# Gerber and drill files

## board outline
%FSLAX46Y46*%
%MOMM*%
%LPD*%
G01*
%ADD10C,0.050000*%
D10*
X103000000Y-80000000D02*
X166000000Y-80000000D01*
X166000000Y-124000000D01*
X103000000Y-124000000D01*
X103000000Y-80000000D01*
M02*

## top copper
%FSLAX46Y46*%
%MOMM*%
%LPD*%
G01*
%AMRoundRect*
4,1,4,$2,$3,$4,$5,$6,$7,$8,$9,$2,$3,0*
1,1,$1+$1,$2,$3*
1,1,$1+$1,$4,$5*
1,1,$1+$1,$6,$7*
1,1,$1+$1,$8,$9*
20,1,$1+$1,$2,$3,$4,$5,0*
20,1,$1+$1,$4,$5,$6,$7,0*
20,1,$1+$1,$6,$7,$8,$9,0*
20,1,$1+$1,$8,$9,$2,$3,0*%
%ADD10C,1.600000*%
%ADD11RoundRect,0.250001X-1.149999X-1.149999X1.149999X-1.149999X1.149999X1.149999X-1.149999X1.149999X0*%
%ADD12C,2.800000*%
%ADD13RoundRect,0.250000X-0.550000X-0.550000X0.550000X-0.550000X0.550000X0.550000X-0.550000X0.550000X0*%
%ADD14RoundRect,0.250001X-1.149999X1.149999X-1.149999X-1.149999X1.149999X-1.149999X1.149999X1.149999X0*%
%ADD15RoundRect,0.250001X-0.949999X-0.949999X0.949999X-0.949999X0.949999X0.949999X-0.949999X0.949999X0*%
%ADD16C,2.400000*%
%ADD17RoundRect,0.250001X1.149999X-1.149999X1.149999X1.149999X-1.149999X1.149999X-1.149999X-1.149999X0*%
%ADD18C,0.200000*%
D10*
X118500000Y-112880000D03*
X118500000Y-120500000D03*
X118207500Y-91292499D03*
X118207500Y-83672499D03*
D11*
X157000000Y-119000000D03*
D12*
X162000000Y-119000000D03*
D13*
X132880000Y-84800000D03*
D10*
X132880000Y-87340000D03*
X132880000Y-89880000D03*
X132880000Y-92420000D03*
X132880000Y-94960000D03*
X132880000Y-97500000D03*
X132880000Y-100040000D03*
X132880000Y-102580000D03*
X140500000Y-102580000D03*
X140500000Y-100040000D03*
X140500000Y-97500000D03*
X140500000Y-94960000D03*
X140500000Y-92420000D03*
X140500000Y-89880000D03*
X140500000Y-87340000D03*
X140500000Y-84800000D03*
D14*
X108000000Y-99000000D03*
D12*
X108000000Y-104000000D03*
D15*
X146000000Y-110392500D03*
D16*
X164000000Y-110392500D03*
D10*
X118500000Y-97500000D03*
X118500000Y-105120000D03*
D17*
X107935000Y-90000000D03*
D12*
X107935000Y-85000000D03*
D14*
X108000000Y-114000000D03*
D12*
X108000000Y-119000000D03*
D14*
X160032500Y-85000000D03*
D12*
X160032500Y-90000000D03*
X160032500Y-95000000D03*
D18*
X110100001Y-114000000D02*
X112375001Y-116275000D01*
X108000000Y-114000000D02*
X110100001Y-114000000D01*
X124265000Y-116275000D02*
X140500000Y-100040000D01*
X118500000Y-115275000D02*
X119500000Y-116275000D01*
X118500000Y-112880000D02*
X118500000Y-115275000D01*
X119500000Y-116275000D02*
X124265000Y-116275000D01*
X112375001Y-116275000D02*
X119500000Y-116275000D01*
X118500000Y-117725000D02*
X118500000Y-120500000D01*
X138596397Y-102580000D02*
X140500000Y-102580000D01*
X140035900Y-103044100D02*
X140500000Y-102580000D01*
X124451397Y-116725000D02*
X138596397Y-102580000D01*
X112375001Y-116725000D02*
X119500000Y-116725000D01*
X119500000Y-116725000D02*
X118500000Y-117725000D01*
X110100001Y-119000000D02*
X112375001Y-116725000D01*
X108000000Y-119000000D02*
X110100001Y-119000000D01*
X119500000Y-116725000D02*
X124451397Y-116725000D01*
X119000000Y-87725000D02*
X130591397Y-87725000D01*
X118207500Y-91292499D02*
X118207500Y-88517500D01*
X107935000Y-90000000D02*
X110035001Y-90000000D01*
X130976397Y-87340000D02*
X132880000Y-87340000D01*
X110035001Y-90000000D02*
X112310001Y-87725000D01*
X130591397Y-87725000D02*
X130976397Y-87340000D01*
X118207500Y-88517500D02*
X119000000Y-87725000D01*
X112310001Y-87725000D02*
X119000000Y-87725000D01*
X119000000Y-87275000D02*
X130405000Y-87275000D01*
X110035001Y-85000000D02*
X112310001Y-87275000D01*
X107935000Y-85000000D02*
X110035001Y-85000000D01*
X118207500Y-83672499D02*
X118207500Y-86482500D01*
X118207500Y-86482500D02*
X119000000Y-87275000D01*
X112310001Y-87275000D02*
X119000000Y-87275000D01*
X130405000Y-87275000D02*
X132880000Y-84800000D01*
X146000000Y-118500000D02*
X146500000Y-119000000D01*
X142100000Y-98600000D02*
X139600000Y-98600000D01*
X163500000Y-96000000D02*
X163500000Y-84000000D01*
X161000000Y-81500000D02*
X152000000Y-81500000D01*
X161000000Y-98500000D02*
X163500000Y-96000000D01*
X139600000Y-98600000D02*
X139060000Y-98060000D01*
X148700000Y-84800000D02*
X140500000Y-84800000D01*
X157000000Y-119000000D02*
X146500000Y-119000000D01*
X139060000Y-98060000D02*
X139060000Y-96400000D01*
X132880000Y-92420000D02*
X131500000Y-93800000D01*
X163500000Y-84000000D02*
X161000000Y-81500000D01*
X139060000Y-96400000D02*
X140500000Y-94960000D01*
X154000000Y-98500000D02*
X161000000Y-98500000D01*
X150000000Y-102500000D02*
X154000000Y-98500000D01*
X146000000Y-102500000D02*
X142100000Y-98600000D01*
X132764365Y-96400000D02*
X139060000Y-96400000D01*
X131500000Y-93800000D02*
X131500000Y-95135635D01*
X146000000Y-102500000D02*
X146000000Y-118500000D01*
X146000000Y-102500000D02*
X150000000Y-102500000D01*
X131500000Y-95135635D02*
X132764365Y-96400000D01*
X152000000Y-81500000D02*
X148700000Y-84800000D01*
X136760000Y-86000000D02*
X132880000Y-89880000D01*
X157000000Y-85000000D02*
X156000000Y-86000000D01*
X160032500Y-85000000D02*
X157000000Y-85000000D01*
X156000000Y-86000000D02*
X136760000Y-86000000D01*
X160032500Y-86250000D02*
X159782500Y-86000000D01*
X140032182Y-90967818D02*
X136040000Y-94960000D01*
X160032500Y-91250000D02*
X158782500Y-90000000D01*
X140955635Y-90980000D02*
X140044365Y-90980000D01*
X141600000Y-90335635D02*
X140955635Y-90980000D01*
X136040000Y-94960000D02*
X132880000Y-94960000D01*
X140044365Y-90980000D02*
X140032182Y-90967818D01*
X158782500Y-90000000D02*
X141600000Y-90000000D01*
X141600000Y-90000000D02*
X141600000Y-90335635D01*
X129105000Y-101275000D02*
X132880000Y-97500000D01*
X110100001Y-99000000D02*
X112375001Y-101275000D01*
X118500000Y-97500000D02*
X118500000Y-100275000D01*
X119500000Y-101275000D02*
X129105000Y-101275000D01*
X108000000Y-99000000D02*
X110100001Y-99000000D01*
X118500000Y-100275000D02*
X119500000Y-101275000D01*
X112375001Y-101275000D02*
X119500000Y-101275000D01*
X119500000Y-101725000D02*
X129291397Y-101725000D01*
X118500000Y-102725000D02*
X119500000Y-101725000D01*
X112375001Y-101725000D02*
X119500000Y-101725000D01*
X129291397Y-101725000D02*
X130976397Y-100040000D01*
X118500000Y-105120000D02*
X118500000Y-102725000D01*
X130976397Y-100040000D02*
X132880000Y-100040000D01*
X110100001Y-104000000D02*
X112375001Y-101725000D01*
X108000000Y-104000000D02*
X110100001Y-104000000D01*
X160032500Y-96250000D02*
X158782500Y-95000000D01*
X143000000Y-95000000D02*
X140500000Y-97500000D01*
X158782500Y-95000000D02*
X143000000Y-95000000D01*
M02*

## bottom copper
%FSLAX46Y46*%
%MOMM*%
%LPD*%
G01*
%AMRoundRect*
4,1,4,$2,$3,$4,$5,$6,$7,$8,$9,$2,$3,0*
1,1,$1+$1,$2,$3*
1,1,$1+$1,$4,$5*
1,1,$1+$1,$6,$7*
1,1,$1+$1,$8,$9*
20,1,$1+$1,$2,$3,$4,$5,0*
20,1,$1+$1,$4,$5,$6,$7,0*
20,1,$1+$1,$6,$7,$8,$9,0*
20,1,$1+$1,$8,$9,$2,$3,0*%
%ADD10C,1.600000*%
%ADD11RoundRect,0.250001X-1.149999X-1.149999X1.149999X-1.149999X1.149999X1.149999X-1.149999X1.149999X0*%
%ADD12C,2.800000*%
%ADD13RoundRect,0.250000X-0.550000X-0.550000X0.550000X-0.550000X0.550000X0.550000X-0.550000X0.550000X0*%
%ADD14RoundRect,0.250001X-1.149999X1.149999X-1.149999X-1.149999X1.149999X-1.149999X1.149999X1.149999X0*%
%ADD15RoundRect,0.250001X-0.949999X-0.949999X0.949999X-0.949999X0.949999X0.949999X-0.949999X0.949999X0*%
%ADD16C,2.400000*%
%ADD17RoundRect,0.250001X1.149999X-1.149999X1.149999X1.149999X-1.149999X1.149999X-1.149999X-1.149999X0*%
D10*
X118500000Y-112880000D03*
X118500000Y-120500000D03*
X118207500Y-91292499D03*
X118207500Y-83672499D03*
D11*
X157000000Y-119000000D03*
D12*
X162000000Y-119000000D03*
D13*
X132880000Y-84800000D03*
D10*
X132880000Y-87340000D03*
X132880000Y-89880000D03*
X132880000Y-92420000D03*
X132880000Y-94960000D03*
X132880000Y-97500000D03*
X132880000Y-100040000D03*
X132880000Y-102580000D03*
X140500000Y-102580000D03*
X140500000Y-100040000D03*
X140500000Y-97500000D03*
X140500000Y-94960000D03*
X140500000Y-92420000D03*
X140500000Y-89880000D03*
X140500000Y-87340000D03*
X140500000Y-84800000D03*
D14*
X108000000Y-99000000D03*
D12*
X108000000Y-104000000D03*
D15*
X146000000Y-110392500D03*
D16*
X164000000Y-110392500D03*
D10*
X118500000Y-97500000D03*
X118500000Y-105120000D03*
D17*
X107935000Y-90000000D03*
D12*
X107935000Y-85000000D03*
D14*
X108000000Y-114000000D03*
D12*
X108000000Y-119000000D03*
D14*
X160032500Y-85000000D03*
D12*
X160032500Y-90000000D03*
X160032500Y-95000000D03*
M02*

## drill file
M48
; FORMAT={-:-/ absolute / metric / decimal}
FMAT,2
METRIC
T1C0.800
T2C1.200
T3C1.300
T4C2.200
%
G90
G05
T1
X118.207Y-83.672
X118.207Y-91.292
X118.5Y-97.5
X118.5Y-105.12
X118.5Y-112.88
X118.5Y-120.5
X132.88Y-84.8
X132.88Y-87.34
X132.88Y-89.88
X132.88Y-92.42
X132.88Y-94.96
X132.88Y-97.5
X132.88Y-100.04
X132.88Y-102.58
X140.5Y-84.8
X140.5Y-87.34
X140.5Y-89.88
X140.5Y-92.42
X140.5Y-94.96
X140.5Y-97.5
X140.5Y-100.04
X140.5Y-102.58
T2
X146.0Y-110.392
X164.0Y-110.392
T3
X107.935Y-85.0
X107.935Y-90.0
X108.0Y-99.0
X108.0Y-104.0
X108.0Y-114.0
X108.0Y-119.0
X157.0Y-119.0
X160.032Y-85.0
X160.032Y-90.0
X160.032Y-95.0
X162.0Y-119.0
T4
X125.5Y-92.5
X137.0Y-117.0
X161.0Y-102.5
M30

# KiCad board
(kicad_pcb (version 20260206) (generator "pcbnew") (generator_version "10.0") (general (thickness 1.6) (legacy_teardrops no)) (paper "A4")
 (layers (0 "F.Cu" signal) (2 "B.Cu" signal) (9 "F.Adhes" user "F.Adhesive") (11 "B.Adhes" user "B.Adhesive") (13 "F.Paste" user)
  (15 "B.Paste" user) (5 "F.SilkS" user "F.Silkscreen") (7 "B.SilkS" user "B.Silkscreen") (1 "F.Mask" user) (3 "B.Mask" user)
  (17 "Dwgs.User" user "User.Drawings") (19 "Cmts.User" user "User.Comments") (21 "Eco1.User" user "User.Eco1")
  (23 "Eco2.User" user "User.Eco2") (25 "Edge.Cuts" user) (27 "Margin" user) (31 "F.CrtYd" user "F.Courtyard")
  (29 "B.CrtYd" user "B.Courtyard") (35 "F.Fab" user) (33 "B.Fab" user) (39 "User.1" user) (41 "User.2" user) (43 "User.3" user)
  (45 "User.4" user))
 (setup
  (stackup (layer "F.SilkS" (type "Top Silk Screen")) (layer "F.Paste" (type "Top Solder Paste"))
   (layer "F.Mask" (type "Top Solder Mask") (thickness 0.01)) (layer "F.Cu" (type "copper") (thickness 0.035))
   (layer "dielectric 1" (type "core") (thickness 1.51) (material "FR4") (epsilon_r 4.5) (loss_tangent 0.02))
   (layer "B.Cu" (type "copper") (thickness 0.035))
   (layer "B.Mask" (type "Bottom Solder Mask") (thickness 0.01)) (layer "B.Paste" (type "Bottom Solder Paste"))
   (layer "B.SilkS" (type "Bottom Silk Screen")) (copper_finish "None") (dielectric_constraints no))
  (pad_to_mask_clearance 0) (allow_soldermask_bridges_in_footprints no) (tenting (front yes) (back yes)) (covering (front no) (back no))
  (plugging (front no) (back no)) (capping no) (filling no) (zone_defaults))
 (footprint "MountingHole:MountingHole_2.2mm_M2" (layer "F.Cu") (at 125.5 92.5)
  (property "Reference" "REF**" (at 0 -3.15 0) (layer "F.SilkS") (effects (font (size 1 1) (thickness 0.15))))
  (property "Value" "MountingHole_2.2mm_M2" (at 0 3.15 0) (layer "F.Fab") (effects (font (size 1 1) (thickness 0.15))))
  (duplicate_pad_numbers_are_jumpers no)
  (pad "" np_thru_hole circle (at 0 0) (size 2.2 2.2) (drill 2.2) (layers "*.Cu" "*.Mask")))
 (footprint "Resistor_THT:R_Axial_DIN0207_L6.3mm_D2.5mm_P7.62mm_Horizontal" (layer "F.Cu") (at 118.5 112.88 -90)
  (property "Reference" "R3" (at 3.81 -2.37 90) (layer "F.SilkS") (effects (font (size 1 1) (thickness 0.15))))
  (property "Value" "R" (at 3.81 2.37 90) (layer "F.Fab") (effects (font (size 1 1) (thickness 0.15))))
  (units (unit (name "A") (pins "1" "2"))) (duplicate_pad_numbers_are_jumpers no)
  (pad "1" thru_hole circle (at 0 0 270) (size 1.6 1.6) (drill 0.8) (layers "*.Cu" "*.Mask") (remove_unused_layers no) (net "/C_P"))
  (pad "2" thru_hole circle (at 7.62 0 270) (size 1.6 1.6) (drill 0.8) (layers "*.Cu" "*.Mask") (remove_unused_layers no) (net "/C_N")))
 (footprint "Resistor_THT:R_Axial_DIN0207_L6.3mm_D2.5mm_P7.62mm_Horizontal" (layer "F.Cu") (at 118.2075 91.292499 90)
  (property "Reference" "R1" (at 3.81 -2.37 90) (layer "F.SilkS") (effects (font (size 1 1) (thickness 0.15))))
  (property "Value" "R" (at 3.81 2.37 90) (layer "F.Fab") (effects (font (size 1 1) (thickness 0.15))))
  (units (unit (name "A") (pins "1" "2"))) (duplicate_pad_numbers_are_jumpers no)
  (pad "1" thru_hole circle (at 0 0 90) (size 1.6 1.6) (drill 0.8) (layers "*.Cu" "*.Mask") (remove_unused_layers no) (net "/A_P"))
  (pad "2" thru_hole circle (at 7.62 0 90) (size 1.6 1.6) (drill 0.8) (layers "*.Cu" "*.Mask") (remove_unused_layers no) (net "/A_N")))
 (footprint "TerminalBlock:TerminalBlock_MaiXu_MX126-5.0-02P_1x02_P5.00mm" (layer "F.Cu") (at 157 119)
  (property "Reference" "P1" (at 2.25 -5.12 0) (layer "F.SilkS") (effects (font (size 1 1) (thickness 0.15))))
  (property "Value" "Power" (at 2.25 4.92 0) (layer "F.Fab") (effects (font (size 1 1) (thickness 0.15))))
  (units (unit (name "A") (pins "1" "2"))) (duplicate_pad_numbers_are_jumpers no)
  (pad "1" thru_hole roundrect (at 0 0) (size 2.8 2.8) (drill 1.3) (layers "*.Cu" "*.Mask") (remove_unused_layers no)
   (roundrect_rratio 0.089286) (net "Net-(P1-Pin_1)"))
  (pad "2" thru_hole circle (at 5 0) (size 2.8 2.8) (drill 1.3) (layers "*.Cu" "*.Mask") (remove_unused_layers no) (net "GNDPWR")))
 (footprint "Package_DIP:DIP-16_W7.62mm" (layer "F.Cu") (at 132.88 84.8)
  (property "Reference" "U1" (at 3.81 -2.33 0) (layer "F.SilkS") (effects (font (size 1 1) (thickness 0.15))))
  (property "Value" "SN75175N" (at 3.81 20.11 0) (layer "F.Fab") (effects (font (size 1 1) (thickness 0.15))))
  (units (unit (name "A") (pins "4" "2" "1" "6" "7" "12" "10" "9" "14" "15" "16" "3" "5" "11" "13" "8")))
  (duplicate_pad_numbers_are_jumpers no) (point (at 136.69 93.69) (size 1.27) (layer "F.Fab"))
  (pad "1" thru_hole roundrect (at 0 0) (size 1.6 1.6) (drill 0.8) (layers "*.Cu" "*.Mask") (remove_unused_layers no)
   (roundrect_rratio 0.15625) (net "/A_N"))
  (pad "2" thru_hole circle (at 0 2.54) (size 1.6 1.6) (drill 0.8) (layers "*.Cu" "*.Mask") (remove_unused_layers no) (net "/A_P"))
  (pad "3" thru_hole circle (at 0 5.08) (size 1.6 1.6) (drill 0.8) (layers "*.Cu" "*.Mask") (remove_unused_layers no) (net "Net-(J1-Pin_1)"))
  (pad "4" thru_hole circle (at 0 7.62) (size 1.6 1.6) (drill 0.8) (layers "*.Cu" "*.Mask") (remove_unused_layers no) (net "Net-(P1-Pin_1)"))
  (pad "5" thru_hole circle (at 0 10.16) (size 1.6 1.6) (drill 0.8) (layers "*.Cu" "*.Mask") (remove_unused_layers no)
   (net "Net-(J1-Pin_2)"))
  (pad "6" thru_hole circle (at 0 12.7) (size 1.6 1.6) (drill 0.8) (layers "*.Cu" "*.Mask") (remove_unused_layers no) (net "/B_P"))
  (pad "7" thru_hole circle (at 0 15.24) (size 1.6 1.6) (drill 0.8) (layers "*.Cu" "*.Mask") (remove_unused_layers no) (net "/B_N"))
  (pad "8" thru_hole circle (at 0 17.78) (size 1.6 1.6) (drill 0.8) (layers "*.Cu" "*.Mask") (remove_unused_layers no) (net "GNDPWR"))
  (pad "9" thru_hole circle (at 7.62 17.78) (size 1.6 1.6) (drill 0.8) (layers "*.Cu" "*.Mask") (remove_unused_layers no) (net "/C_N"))
  (pad "10" thru_hole circle (at 7.62 15.24) (size 1.6 1.6) (drill 0.8) (layers "*.Cu" "*.Mask") (remove_unused_layers no) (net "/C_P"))
  (pad "11" thru_hole circle (at 7.62 12.7) (size 1.6 1.6) (drill 0.8) (layers "*.Cu" "*.Mask") (remove_unused_layers no)
   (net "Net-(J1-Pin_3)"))
  (pad "12" thru_hole circle (at 7.62 10.16) (size 1.6 1.6) (drill 0.8) (layers "*.Cu" "*.Mask") (remove_unused_layers no)
   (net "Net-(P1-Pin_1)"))
  (pad "13" thru_hole circle (at 7.62 7.62) (size 1.6 1.6) (drill 0.8) (layers "*.Cu" "*.Mask") (remove_unused_layers no)
   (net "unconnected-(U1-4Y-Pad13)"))
  (pad "14" thru_hole circle (at 7.62 5.08) (size 1.6 1.6) (drill 0.8) (layers "*.Cu" "*.Mask") (remove_unused_layers no)
   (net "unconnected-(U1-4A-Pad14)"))
  (pad "15" thru_hole circle (at 7.62 2.54) (size 1.6 1.6) (drill 0.8) (layers "*.Cu" "*.Mask") (remove_unused_layers no)
   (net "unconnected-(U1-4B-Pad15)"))
  (pad "16" thru_hole circle (at 7.62 0) (size 1.6 1.6) (drill 0.8) (layers "*.Cu" "*.Mask") (remove_unused_layers no)
   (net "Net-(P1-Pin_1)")))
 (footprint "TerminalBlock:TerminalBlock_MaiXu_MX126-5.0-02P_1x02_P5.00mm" (layer "F.Cu") (at 108 99 -90)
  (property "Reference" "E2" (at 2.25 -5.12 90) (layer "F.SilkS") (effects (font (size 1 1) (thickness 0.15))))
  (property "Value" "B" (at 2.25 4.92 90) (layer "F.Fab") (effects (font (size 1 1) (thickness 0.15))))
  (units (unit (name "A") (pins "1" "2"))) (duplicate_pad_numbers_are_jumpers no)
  (pad "1" thru_hole roundrect (at 0 0 270) (size 2.8 2.8) (drill 1.3) (layers "*.Cu" "*.Mask") (remove_unused_layers no)
   (roundrect_rratio 0.089286) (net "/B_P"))
  (pad "2" thru_hole circle (at 5 0 270) (size 2.8 2.8) (drill 1.3) (layers "*.Cu" "*.Mask") (remove_unused_layers no) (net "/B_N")))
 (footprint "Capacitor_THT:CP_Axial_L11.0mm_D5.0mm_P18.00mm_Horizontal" (layer "F.Cu") (at 146 110.3925)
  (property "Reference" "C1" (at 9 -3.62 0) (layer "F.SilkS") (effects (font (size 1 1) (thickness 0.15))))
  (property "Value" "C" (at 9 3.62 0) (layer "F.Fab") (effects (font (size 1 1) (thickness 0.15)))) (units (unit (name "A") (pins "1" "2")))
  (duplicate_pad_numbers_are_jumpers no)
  (pad "1" thru_hole roundrect (at 0 0) (size 2.4 2.4) (drill 1.2) (layers "*.Cu" "*.Mask") (remove_unused_layers no)
   (roundrect_rratio 0.104167) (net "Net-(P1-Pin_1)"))
  (pad "2" thru_hole circle (at 18 0) (size 2.4 2.4) (drill 1.2) (layers "*.Cu" "*.Mask") (remove_unused_layers no) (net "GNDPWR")))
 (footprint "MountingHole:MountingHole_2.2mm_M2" (layer "F.Cu") (at 137 117)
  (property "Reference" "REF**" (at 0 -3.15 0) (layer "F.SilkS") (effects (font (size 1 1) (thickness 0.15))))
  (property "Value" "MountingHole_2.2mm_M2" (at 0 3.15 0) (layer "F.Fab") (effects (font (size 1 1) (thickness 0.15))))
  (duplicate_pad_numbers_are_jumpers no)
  (pad "" np_thru_hole circle (at 0 0) (size 2.2 2.2) (drill 2.2) (layers "*.Cu" "*.Mask")))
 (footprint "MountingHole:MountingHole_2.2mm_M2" (layer "F.Cu") (at 161 102.5)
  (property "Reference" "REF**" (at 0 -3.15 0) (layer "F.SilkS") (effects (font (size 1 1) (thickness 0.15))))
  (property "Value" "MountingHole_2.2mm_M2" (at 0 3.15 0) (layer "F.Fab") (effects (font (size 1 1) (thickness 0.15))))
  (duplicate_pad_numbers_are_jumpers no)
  (pad "" np_thru_hole circle (at 0 0) (size 2.2 2.2) (drill 2.2) (layers "*.Cu" "*.Mask")))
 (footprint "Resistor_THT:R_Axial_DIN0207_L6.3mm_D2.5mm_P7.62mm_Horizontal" (layer "F.Cu") (at 118.5 97.5 -90)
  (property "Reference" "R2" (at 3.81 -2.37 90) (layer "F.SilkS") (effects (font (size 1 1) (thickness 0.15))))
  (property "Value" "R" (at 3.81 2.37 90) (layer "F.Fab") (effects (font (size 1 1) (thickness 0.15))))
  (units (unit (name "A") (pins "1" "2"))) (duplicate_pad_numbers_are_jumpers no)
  (pad "1" thru_hole circle (at 0 0 270) (size 1.6 1.6) (drill 0.8) (layers "*.Cu" "*.Mask") (remove_unused_layers no) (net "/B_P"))
  (pad "2" thru_hole circle (at 7.62 0 270) (size 1.6 1.6) (drill 0.8) (layers "*.Cu" "*.Mask") (remove_unused_layers no) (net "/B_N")))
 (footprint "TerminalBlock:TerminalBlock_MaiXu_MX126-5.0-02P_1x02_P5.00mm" (layer "F.Cu") (at 107.935 90 90)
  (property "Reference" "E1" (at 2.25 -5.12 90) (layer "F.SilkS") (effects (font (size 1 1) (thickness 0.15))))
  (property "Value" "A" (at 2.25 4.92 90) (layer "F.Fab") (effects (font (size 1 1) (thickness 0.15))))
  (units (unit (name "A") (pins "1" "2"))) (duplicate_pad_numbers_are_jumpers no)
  (pad "1" thru_hole roundrect (at 0 0 90) (size 2.8 2.8) (drill 1.3) (layers "*.Cu" "*.Mask") (remove_unused_layers no)
   (roundrect_rratio 0.089286) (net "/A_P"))
  (pad "2" thru_hole circle (at 5 0 90) (size 2.8 2.8) (drill 1.3) (layers "*.Cu" "*.Mask") (remove_unused_layers no) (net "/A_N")))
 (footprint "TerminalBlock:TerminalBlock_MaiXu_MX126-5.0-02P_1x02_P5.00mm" (layer "F.Cu") (at 108 114 -90)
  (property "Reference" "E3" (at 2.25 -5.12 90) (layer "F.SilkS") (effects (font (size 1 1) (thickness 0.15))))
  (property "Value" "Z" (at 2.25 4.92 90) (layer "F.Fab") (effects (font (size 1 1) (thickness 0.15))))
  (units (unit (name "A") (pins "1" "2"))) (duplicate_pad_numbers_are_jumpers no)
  (pad "1" thru_hole roundrect (at 0 0 270) (size 2.8 2.8) (drill 1.3) (layers "*.Cu" "*.Mask") (remove_unused_layers no)
   (roundrect_rratio 0.089286) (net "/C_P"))
  (pad "2" thru_hole circle (at 5 0 270) (size 2.8 2.8) (drill 1.3) (layers "*.Cu" "*.Mask") (remove_unused_layers no) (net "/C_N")))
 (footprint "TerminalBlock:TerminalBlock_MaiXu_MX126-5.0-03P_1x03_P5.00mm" (layer "F.Cu") (at 160.0325 85 -90)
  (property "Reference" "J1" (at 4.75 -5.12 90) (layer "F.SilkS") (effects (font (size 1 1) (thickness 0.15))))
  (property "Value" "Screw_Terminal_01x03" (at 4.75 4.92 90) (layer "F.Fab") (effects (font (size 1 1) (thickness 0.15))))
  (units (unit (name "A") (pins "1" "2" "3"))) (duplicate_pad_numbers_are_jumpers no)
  (pad "1" thru_hole roundrect (at 0 0 270) (size 2.8 2.8) (drill 1.3) (layers "*.Cu" "*.Mask") (remove_unused_layers no)
   (roundrect_rratio 0.089286) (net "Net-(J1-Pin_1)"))
  (pad "2" thru_hole circle (at 5 0 270) (size 2.8 2.8) (drill 1.3) (layers "*.Cu" "*.Mask") (remove_unused_layers no)
   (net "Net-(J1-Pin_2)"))
  (pad "3" thru_hole circle (at 10 0 270) (size 2.8 2.8) (drill 1.3) (layers "*.Cu" "*.Mask") (remove_unused_layers no)
   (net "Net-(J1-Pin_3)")))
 (gr_rect (start 103 80) (end 166 124) (stroke (width 0.05) (type default)) (fill no) (layer "Edge.Cuts"))
 (segment (start 110.100001 114) (end 112.375001 116.275) (width 0.2) (layer "F.Cu") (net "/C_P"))
 (segment (start 108 114) (end 110.100001 114) (width 0.2) (layer "F.Cu") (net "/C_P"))
 (segment (start 124.265 116.275) (end 140.5 100.04) (width 0.2) (layer "F.Cu") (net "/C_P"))
 (segment (start 118.5 115.275) (end 119.5 116.275) (width 0.2) (layer "F.Cu") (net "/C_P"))
 (segment (start 118.5 112.88) (end 118.5 115.275) (width 0.2) (layer "F.Cu") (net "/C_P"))
 (segment (start 119.5 116.275) (end 124.265 116.275) (width 0.2) (layer "F.Cu") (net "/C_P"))
 (segment (start 112.375001 116.275) (end 119.5 116.275) (width 0.2) (layer "F.Cu") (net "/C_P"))
 (segment (start 118.5 117.725) (end 118.5 120.5) (width 0.2) (layer "F.Cu") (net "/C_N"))
 (segment (start 138.596397 102.58) (end 140.5 102.58) (width 0.2) (layer "F.Cu") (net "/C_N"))
 (segment (start 140.0359 103.0441) (end 140.5 102.58) (width 0.2) (layer "F.Cu") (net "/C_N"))
 (segment (start 124.451397 116.725) (end 138.596397 102.58) (width 0.2) (layer "F.Cu") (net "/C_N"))
 (segment (start 112.375001 116.725) (end 119.5 116.725) (width 0.2) (layer "F.Cu") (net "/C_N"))
 (segment (start 119.5 116.725) (end 118.5 117.725) (width 0.2) (layer "F.Cu") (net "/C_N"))
 (segment (start 110.100001 119) (end 112.375001 116.725) (width 0.2) (layer "F.Cu") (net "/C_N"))
 (segment (start 108 119) (end 110.100001 119) (width 0.2) (layer "F.Cu") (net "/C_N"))
 (segment (start 119.5 116.725) (end 124.451397 116.725) (width 0.2) (layer "F.Cu") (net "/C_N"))
 (segment (start 119 87.725) (end 130.591397 87.725) (width 0.2) (layer "F.Cu") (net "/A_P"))
 (segment (start 118.2075 91.292499) (end 118.2075 88.5175) (width 0.2) (layer "F.Cu") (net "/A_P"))
 (segment (start 107.935 90) (end 110.035001 90) (width 0.2) (layer "F.Cu") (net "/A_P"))
 (segment (start 130.976397 87.34) (end 132.88 87.34) (width 0.2) (layer "F.Cu") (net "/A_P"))
 (segment (start 110.035001 90) (end 112.310001 87.725) (width 0.2) (layer "F.Cu") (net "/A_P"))
 (segment (start 130.591397 87.725) (end 130.976397 87.34) (width 0.2) (layer "F.Cu") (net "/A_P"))
 (segment (start 118.2075 88.5175) (end 119 87.725) (width 0.2) (layer "F.Cu") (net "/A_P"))
 (segment (start 112.310001 87.725) (end 119 87.725) (width 0.2) (layer "F.Cu") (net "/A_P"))
 (segment (start 119 87.275) (end 130.405 87.275) (width 0.2) (layer "F.Cu") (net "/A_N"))
 (segment (start 110.035001 85) (end 112.310001 87.275) (width 0.2) (layer "F.Cu") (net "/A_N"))
 (segment (start 107.935 85) (end 110.035001 85) (width 0.2) (layer "F.Cu") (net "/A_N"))
 (segment (start 118.2075 83.672499) (end 118.2075 86.4825) (width 0.2) (layer "F.Cu") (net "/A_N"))
 (segment (start 118.2075 86.4825) (end 119 87.275) (width 0.2) (layer "F.Cu") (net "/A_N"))
 (segment (start 112.310001 87.275) (end 119 87.275) (width 0.2) (layer "F.Cu") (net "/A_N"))
 (segment (start 130.405 87.275) (end 132.88 84.8) (width 0.2) (layer "F.Cu") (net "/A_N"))
 (segment (start 146 118.5) (end 146.5 119) (width 0.2) (layer "F.Cu") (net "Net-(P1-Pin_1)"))
 (segment (start 142.1 98.6) (end 139.6 98.6) (width 0.2) (layer "F.Cu") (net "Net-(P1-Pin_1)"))
 (segment (start 163.5 96) (end 163.5 84) (width 0.2) (layer "F.Cu") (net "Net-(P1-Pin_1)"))
 (segment (start 161 81.5) (end 152 81.5) (width 0.2) (layer "F.Cu") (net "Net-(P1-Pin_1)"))
 (segment (start 161 98.5) (end 163.5 96) (width 0.2) (layer "F.Cu") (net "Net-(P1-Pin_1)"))
 (segment (start 139.6 98.6) (end 139.06 98.06) (width 0.2) (layer "F.Cu") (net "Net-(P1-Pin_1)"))
 (segment (start 148.7 84.8) (end 140.5 84.8) (width 0.2) (layer "F.Cu") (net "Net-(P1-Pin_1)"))
 (segment (start 157 119) (end 146.5 119) (width 0.2) (layer "F.Cu") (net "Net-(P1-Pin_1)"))
 (segment (start 139.06 98.06) (end 139.06 96.4) (width 0.2) (layer "F.Cu") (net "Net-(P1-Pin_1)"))
 (segment (start 132.88 92.42) (end 131.5 93.8) (width 0.2) (layer "F.Cu") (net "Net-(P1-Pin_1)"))
 (segment (start 163.5 84) (end 161 81.5) (width 0.2) (layer "F.Cu") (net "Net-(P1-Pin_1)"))
 (segment (start 139.06 96.4) (end 140.5 94.96) (width 0.2) (layer "F.Cu") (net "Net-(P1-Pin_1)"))
 (segment (start 154 98.5) (end 161 98.5) (width 0.2) (layer "F.Cu") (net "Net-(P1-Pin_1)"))
 (segment (start 150 102.5) (end 154 98.5) (width 0.2) (layer "F.Cu") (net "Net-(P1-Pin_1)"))
 (segment (start 146 102.5) (end 142.1 98.6) (width 0.2) (layer "F.Cu") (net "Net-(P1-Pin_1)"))
 (segment (start 132.764365 96.4) (end 139.06 96.4) (width 0.2) (layer "F.Cu") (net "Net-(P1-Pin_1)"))
 (segment (start 131.5 93.8) (end 131.5 95.135635) (width 0.2) (layer "F.Cu") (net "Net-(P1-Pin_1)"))
 (segment (start 146 102.5) (end 146 118.5) (width 0.2) (layer "F.Cu") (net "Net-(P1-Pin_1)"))
 (segment (start 146 102.5) (end 150 102.5) (width 0.2) (layer "F.Cu") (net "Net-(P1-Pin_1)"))
 (segment (start 131.5 95.135635) (end 132.764365 96.4) (width 0.2) (layer "F.Cu") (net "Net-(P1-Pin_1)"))
 (segment (start 152 81.5) (end 148.7 84.8) (width 0.2) (layer "F.Cu") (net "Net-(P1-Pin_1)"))
 (segment (start 136.76 86) (end 132.88 89.88) (width 0.2) (layer "F.Cu") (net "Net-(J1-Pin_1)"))
 (segment (start 157 85) (end 156 86) (width 0.2) (layer "F.Cu") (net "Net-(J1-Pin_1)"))
 (segment (start 160.0325 85) (end 157 85) (width 0.2) (layer "F.Cu") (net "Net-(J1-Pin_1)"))
 (segment (start 156 86) (end 136.76 86) (width 0.2) (layer "F.Cu") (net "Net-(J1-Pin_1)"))
 (segment (start 160.0325 86.25) (end 159.7825 86) (width 0.2) (layer "F.Cu") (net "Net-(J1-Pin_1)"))
 (segment (start 140.032182 90.967818) (end 136.04 94.96) (width 0.2) (layer "F.Cu") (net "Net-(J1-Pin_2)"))
 (segment (start 160.0325 91.25) (end 158.7825 90) (width 0.2) (layer "F.Cu") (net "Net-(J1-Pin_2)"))
 (segment (start 140.955635 90.98) (end 140.044365 90.98) (width 0.2) (layer "F.Cu") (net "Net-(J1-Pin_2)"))
 (segment (start 141.6 90.335635) (end 140.955635 90.98) (width 0.2) (layer "F.Cu") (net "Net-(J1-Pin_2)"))
 (segment (start 136.04 94.96) (end 132.88 94.96) (width 0.2) (layer "F.Cu") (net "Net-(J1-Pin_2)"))
 (segment (start 140.044365 90.98) (end 140.032182 90.967818) (width 0.2) (layer "F.Cu") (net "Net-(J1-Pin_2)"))
 (segment (start 158.7825 90) (end 141.6 90) (width 0.2) (layer "F.Cu") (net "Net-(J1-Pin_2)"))
 (segment (start 141.6 90) (end 141.6 90.335635) (width 0.2) (layer "F.Cu") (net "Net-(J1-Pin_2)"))
 (segment (start 129.105 101.275) (end 132.88 97.5) (width 0.2) (layer "F.Cu") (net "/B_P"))
 (segment (start 110.100001 99) (end 112.375001 101.275) (width 0.2) (layer "F.Cu") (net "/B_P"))
 (segment (start 118.5 97.5) (end 118.5 100.275) (width 0.2) (layer "F.Cu") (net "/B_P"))
 (segment (start 119.5 101.275) (end 129.105 101.275) (width 0.2) (layer "F.Cu") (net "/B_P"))
 (segment (start 108 99) (end 110.100001 99) (width 0.2) (layer "F.Cu") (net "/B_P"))
 (segment (start 118.5 100.275) (end 119.5 101.275) (width 0.2) (layer "F.Cu") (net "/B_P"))
 (segment (start 112.375001 101.275) (end 119.5 101.275) (width 0.2) (layer "F.Cu") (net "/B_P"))
 (segment (start 119.5 101.725) (end 129.291397 101.725) (width 0.2) (layer "F.Cu") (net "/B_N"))
 (segment (start 118.5 102.725) (end 119.5 101.725) (width 0.2) (layer "F.Cu") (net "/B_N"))
 (segment (start 112.375001 101.725) (end 119.5 101.725) (width 0.2) (layer "F.Cu") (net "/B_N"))
 (segment (start 129.291397 101.725) (end 130.976397 100.04) (width 0.2) (layer "F.Cu") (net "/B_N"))
 (segment (start 118.5 105.12) (end 118.5 102.725) (width 0.2) (layer "F.Cu") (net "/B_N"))
 (segment (start 130.976397 100.04) (end 132.88 100.04) (width 0.2) (layer "F.Cu") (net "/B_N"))
 (segment (start 110.100001 104) (end 112.375001 101.725) (width 0.2) (layer "F.Cu") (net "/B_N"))
 (segment (start 108 104) (end 110.100001 104) (width 0.2) (layer "F.Cu") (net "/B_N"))
 (segment (start 160.0325 96.25) (end 158.7825 95) (width 0.2) (layer "F.Cu") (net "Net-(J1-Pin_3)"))
 (segment (start 143 95) (end 140.5 97.5) (width 0.2) (layer "F.Cu") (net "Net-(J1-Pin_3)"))
 (segment (start 158.7825 95) (end 143 95) (width 0.2) (layer "F.Cu") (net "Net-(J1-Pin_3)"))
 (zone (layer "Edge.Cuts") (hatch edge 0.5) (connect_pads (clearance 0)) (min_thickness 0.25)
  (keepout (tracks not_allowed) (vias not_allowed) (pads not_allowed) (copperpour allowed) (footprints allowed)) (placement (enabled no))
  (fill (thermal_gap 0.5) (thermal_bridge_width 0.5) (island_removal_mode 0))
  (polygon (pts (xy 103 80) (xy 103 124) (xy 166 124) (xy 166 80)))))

